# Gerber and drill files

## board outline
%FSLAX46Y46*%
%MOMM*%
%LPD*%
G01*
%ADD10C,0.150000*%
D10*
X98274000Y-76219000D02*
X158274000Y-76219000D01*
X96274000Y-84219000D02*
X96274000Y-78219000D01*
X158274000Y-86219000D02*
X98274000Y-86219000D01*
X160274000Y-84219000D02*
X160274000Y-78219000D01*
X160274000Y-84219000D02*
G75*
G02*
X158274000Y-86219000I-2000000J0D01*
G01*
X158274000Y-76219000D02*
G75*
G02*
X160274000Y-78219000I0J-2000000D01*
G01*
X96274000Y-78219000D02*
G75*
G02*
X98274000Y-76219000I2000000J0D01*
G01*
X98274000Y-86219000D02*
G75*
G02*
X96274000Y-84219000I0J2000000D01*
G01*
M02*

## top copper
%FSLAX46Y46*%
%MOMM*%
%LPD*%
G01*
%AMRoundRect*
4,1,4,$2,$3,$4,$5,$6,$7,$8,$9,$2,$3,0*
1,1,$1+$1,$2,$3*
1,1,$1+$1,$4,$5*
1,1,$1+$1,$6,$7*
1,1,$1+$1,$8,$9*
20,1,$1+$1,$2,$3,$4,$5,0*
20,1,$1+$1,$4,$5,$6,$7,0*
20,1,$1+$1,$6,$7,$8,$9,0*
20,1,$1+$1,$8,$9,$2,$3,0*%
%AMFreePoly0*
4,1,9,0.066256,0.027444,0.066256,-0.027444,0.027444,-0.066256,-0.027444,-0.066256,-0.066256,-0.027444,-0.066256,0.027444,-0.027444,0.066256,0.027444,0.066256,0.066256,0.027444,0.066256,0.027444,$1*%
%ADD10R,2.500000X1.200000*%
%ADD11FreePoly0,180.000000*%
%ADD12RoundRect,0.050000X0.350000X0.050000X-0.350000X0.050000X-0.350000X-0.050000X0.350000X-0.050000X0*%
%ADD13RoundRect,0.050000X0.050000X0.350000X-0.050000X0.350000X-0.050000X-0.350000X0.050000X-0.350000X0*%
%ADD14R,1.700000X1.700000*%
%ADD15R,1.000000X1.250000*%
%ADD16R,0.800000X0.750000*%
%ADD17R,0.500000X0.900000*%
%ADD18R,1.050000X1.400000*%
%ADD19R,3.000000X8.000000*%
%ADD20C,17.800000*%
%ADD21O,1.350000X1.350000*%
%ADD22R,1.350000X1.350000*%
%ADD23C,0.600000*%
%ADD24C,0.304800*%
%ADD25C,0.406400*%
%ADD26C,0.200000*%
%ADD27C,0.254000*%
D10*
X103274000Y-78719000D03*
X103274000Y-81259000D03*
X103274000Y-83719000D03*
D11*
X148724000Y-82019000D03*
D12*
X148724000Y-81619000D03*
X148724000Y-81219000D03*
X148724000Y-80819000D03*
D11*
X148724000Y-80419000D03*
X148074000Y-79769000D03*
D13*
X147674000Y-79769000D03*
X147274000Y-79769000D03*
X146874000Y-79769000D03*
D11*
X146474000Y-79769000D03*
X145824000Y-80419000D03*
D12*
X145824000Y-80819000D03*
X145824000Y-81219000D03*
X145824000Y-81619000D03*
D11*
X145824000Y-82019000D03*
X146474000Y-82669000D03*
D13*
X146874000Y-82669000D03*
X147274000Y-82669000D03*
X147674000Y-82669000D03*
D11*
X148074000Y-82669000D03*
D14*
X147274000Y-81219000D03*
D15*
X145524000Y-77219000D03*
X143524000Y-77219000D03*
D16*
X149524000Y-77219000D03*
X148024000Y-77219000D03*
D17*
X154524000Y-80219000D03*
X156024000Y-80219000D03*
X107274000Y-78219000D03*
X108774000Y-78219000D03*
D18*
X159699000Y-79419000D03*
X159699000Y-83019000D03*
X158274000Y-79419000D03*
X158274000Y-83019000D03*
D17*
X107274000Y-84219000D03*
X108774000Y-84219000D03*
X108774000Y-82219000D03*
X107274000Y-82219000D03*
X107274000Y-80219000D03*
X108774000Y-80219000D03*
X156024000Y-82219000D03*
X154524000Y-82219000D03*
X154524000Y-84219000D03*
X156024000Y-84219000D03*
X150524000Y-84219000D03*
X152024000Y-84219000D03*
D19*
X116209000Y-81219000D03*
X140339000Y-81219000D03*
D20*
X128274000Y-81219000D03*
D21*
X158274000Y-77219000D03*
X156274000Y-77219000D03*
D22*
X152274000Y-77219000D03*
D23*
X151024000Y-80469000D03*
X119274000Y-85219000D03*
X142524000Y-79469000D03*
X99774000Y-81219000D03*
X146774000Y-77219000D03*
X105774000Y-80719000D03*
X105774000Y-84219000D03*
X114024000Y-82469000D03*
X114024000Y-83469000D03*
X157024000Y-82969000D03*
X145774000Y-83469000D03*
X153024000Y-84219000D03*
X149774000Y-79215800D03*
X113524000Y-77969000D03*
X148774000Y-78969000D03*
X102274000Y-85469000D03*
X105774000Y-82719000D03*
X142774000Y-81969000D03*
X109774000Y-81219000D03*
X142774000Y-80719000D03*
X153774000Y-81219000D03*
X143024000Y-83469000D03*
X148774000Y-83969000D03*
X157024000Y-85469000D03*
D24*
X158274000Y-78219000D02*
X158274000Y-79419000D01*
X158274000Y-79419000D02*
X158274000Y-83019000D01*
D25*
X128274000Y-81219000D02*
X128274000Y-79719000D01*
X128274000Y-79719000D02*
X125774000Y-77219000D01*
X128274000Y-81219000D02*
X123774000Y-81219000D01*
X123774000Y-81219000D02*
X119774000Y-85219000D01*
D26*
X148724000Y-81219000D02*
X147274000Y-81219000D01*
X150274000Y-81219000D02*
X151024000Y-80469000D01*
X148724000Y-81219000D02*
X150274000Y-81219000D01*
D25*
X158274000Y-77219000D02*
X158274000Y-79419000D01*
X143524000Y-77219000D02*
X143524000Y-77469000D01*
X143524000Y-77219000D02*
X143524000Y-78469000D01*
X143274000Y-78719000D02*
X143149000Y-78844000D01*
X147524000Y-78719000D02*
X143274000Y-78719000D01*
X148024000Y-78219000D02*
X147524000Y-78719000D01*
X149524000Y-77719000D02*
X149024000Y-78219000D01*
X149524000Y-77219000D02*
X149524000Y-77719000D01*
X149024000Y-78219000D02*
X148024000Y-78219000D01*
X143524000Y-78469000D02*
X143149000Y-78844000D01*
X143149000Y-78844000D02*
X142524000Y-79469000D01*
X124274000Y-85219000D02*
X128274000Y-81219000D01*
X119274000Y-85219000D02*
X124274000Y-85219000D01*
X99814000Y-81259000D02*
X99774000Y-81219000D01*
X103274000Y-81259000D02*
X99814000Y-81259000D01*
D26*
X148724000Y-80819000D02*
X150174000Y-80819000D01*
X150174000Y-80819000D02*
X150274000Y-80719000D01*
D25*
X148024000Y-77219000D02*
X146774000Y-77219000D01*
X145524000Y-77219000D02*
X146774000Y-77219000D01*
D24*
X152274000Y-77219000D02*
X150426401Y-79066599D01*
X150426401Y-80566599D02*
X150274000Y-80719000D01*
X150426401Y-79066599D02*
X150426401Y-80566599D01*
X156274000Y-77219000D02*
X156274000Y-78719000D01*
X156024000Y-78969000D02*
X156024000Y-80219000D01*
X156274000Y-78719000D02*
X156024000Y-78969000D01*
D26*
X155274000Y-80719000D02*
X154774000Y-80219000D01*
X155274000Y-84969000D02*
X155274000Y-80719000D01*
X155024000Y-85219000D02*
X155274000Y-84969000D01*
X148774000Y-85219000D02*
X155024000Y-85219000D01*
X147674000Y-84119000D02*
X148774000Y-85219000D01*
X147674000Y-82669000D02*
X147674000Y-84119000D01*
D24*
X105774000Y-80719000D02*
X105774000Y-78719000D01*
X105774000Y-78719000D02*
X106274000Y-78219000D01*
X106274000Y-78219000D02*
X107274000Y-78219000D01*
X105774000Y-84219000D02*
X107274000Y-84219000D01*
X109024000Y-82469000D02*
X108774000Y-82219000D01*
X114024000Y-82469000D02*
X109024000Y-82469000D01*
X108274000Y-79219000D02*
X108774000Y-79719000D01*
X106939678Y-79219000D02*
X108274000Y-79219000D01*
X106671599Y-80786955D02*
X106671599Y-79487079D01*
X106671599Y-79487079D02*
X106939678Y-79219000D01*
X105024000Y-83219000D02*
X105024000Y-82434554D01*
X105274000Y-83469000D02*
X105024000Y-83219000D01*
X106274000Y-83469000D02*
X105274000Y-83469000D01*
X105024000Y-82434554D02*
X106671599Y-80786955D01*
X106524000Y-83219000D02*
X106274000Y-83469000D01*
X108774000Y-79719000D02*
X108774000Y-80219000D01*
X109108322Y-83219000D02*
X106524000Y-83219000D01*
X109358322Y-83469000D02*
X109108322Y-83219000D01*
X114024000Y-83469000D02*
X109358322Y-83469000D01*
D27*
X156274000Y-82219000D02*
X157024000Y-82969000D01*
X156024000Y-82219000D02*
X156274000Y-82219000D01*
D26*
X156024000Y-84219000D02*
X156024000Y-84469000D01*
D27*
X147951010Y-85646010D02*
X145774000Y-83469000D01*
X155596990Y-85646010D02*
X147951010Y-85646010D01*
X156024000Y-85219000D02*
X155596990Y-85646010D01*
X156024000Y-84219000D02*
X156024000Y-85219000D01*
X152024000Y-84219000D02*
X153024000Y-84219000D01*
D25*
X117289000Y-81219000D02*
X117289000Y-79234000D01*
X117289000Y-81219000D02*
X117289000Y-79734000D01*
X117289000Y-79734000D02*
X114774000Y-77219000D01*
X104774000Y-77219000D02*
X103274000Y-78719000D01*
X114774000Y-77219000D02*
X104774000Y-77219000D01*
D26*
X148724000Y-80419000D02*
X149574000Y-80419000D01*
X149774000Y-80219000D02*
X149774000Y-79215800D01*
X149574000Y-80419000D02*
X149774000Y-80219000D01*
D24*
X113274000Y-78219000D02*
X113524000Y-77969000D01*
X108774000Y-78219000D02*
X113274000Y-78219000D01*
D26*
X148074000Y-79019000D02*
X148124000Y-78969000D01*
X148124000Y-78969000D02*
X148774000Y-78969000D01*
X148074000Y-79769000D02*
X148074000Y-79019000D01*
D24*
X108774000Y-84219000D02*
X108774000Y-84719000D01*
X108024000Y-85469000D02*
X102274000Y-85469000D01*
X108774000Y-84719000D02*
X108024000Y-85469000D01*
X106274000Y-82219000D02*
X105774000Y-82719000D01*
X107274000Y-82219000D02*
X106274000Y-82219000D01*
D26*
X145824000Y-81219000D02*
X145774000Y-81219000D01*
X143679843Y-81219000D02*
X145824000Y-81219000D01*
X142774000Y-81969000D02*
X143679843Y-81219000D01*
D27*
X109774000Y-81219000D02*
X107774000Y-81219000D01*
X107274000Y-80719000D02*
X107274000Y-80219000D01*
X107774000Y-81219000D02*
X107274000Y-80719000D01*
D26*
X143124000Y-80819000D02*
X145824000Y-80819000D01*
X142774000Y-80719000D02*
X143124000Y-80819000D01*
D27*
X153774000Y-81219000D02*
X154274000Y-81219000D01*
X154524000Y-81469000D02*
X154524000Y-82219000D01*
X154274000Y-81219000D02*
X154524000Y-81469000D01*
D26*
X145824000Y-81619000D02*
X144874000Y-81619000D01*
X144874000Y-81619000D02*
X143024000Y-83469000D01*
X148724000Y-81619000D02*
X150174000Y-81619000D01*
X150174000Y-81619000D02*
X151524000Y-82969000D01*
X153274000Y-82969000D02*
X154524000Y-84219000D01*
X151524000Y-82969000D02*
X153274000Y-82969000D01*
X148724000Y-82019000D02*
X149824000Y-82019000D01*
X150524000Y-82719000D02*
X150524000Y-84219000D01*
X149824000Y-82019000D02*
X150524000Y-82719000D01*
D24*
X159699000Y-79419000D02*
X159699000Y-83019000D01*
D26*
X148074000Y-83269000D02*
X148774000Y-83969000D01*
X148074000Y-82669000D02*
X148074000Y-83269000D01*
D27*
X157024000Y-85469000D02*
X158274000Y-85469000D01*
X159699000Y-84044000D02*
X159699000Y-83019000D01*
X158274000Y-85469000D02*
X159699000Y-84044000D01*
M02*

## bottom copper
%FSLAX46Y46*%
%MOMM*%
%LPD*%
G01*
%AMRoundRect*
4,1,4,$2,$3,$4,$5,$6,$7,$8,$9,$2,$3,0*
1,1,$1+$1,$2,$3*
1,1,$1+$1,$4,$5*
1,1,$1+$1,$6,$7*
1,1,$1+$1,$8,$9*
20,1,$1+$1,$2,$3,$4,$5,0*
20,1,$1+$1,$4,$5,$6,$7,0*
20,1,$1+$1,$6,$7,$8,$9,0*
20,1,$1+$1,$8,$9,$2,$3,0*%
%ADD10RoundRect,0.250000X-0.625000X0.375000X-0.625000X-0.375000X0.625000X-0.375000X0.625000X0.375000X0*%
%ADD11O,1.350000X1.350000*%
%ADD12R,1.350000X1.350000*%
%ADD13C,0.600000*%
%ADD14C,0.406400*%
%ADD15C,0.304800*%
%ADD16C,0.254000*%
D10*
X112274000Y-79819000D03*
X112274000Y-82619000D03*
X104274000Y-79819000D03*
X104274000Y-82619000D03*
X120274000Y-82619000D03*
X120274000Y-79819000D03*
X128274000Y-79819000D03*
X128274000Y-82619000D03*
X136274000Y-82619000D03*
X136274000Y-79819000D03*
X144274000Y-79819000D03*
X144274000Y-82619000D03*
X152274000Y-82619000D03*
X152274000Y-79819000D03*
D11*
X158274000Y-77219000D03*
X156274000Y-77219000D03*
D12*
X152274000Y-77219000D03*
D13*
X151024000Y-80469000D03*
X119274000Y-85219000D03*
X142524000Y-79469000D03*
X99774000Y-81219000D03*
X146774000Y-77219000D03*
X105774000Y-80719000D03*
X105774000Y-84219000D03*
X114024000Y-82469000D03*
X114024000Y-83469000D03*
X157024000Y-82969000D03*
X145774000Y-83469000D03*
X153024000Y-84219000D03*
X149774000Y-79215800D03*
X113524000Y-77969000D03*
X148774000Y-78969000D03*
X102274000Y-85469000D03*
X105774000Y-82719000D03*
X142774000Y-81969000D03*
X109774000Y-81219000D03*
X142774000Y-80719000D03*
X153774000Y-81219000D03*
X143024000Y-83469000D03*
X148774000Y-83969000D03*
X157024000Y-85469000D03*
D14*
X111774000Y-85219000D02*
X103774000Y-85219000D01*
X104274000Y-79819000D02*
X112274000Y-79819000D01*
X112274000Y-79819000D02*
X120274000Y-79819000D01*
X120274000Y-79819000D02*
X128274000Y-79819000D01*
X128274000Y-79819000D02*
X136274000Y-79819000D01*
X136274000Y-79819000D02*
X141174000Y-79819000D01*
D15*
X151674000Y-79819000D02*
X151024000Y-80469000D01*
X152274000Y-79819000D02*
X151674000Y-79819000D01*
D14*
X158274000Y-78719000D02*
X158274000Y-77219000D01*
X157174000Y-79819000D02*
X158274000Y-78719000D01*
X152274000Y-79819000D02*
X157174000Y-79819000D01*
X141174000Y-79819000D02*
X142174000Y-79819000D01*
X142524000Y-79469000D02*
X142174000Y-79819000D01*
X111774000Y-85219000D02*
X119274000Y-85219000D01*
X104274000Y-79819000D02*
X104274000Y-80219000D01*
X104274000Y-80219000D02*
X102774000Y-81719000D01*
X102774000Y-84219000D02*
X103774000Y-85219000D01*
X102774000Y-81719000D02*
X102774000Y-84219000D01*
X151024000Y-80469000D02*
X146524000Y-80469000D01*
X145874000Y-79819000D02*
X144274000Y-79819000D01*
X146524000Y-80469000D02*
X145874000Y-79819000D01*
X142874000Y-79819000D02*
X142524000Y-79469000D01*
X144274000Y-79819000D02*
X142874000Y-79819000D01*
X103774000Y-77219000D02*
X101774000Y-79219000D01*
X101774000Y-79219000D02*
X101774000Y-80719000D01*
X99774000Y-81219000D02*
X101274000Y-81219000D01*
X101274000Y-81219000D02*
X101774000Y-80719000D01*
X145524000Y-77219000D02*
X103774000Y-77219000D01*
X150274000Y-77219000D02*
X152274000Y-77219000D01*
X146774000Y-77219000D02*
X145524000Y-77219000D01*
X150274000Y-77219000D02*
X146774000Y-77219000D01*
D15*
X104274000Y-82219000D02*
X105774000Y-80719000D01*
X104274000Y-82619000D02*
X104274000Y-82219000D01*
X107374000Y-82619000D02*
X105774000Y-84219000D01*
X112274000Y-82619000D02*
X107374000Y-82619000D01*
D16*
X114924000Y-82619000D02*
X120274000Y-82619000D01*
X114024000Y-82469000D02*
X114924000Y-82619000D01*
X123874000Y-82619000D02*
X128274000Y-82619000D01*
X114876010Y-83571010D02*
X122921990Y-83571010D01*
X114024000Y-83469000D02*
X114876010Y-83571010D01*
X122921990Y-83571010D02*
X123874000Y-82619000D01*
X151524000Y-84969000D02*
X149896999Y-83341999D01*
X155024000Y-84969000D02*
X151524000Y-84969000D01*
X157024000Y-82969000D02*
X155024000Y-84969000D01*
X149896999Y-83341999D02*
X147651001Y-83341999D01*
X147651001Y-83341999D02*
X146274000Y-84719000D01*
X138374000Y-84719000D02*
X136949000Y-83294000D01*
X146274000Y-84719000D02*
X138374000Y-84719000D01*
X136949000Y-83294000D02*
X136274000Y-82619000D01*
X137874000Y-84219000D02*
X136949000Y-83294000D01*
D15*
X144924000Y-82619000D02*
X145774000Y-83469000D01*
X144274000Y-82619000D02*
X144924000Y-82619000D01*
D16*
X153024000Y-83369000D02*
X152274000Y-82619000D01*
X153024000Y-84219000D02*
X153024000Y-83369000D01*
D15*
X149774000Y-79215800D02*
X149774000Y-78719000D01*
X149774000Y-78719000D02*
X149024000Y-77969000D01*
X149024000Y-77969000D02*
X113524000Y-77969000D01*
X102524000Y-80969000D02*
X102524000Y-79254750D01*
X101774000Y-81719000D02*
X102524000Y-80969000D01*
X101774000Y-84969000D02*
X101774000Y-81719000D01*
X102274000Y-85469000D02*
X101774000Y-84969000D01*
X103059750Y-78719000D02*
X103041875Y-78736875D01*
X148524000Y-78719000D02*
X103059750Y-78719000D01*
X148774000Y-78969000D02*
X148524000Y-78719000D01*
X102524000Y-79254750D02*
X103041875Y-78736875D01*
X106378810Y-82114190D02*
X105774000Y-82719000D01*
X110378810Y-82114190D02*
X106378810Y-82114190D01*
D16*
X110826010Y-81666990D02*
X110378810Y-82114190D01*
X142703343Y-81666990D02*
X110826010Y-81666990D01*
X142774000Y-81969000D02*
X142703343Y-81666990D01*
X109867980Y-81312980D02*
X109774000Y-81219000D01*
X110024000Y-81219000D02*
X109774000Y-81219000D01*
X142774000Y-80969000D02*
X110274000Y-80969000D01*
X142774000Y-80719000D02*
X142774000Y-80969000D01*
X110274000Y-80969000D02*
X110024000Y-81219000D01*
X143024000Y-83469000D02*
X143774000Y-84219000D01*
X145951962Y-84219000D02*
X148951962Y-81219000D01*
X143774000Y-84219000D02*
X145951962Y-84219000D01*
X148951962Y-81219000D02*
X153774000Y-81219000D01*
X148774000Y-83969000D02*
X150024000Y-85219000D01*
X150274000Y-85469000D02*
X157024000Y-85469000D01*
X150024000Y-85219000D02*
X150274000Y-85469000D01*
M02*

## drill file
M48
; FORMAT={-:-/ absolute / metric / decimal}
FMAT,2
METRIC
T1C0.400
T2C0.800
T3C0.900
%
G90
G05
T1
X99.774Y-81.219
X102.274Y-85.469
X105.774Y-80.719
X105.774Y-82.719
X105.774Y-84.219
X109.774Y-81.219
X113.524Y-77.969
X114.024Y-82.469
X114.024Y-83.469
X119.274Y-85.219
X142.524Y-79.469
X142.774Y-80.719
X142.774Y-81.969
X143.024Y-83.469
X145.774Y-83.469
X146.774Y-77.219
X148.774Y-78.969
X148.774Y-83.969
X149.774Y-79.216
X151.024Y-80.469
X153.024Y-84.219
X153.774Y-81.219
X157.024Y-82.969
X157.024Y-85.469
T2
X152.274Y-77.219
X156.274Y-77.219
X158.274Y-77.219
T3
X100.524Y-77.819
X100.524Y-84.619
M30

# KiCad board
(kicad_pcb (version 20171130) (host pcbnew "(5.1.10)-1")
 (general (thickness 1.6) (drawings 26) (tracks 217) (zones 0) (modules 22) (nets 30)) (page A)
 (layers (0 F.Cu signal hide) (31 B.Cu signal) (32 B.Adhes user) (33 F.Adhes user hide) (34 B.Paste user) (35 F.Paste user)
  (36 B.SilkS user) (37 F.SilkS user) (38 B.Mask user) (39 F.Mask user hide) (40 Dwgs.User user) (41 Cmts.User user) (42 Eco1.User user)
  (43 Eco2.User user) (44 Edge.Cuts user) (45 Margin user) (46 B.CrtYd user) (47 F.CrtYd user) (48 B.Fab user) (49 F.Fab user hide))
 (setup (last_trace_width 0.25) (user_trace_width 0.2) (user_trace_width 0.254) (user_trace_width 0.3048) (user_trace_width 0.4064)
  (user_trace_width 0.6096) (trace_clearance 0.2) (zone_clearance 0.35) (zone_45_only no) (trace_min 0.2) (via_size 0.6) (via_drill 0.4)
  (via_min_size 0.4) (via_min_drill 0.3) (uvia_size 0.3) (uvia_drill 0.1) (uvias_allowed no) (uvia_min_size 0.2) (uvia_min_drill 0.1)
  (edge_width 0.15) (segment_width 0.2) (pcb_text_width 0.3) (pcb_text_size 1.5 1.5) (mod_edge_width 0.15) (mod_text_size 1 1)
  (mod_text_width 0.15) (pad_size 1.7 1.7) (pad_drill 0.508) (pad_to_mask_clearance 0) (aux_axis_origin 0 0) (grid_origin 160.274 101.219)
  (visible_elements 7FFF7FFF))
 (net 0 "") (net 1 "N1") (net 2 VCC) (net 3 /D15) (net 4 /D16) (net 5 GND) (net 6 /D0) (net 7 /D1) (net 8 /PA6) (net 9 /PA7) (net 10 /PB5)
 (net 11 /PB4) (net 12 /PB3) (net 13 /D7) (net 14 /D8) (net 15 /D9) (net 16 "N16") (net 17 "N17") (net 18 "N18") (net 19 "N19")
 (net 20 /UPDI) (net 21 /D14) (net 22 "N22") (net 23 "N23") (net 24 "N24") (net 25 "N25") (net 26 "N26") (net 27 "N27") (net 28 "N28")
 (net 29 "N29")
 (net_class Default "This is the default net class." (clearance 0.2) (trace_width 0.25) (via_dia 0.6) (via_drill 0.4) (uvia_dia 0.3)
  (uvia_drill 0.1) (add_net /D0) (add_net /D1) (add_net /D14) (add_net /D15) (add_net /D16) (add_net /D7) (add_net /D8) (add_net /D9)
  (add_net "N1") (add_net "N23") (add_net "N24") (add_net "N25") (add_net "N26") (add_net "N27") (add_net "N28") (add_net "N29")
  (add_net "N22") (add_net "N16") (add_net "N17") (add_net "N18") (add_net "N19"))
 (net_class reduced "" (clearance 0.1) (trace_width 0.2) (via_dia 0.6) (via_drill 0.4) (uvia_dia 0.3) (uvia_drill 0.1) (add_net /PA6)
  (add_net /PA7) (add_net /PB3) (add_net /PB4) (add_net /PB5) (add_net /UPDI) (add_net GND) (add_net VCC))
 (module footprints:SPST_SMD (layer F.Cu) (at 103.274 81.219 270)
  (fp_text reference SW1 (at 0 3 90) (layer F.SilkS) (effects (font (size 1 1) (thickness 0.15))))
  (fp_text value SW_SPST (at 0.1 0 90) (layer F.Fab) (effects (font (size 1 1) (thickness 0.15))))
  (pad "" np_thru_hole circle (at 3.4 2.75 270) (size 0.9 0.9) (drill 0.9) (layers *.Cu *.Mask))
  (pad 1 smd rect (at -2.5 0 270) (size 1.2 2.5) (layers F.Cu F.Paste F.Mask) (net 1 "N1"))
  (pad 2 smd rect (at 0.04 0 270) (size 1.2 2.5) (layers F.Cu F.Paste F.Mask) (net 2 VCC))
  (pad 3 smd rect (at 2.5 0 270) (size 1.2 2.5) (layers F.Cu F.Paste F.Mask))
  (pad "" np_thru_hole circle (at -3.4 2.75 270) (size 0.9 0.9) (drill 0.9) (layers *.Cu *.Mask)))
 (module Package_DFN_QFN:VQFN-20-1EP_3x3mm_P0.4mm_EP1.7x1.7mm (layer F.Cu) (at 147.274 81.219 180)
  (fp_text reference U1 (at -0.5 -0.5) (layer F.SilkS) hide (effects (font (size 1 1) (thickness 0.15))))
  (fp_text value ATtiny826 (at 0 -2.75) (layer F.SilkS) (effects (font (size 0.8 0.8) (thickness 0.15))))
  (pad 1 smd custom (at -1.45 -0.8 180) (size 0.143431 0.143431) (layers F.Cu F.Paste F.Mask) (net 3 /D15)
   (options (clearance outline) (anchor circle)) (primitives))
  (pad 2 smd roundrect (at -1.45 -0.4 180) (size 0.8 0.2) (layers F.Cu F.Paste F.Mask) (roundrect_rratio 0.25) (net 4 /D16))
  (pad 3 smd roundrect (at -1.45 0 180) (size 0.8 0.2) (layers F.Cu F.Paste F.Mask) (roundrect_rratio 0.25) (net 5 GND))
  (pad 4 smd roundrect (at -1.45 0.4 180) (size 0.8 0.2) (layers F.Cu F.Paste F.Mask) (roundrect_rratio 0.25) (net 2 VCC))
  (pad 5 smd custom (at -1.45 0.8 180) (size 0.143431 0.143431) (layers F.Cu F.Paste F.Mask) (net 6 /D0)
   (options (clearance outline) (anchor circle)) (primitives))
  (pad 6 smd custom (at -0.8 1.45 180) (size 0.143431 0.143431) (layers F.Cu F.Paste F.Mask) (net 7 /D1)
   (options (clearance outline) (anchor circle)) (primitives))
  (pad 7 smd roundrect (at -0.4 1.45 180) (size 0.2 0.8) (layers F.Cu F.Paste F.Mask) (roundrect_rratio 0.25) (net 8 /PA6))
  (pad 8 smd roundrect (at 0 1.45 180) (size 0.2 0.8) (layers F.Cu F.Paste F.Mask) (roundrect_rratio 0.25) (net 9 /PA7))
  (pad 9 smd roundrect (at 0.4 1.45 180) (size 0.2 0.8) (layers F.Cu F.Paste F.Mask) (roundrect_rratio 0.25) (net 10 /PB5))
  (pad 10 smd custom (at 0.8 1.45 180) (size 0.143431 0.143431) (layers F.Cu F.Paste F.Mask) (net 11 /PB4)
   (options (clearance outline) (anchor circle)) (primitives))
  (pad 11 smd custom (at 1.45 0.8 180) (size 0.143431 0.143431) (layers F.Cu F.Paste F.Mask) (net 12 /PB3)
   (options (clearance outline) (anchor circle)) (primitives))
  (pad 12 smd roundrect (at 1.45 0.4 180) (size 0.8 0.2) (layers F.Cu F.Paste F.Mask) (roundrect_rratio 0.25) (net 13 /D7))
  (pad 13 smd roundrect (at 1.45 0 180) (size 0.8 0.2) (layers F.Cu F.Paste F.Mask) (roundrect_rratio 0.25) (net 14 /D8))
  (pad 14 smd roundrect (at 1.45 -0.4 180) (size 0.8 0.2) (layers F.Cu F.Paste F.Mask) (roundrect_rratio 0.25) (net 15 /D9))
  (pad 15 smd custom (at 1.45 -0.8 180) (size 0.143431 0.143431) (layers F.Cu F.Paste F.Mask) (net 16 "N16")
   (options (clearance outline) (anchor circle)) (primitives))
  (pad 16 smd custom (at 0.8 -1.45 180) (size 0.143431 0.143431) (layers F.Cu F.Paste F.Mask) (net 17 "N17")
   (options (clearance outline) (anchor circle)) (primitives))
  (pad 17 smd roundrect (at 0.4 -1.45 180) (size 0.2 0.8) (layers F.Cu F.Paste F.Mask) (roundrect_rratio 0.25) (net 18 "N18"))
  (pad 18 smd roundrect (at 0 -1.45 180) (size 0.2 0.8) (layers F.Cu F.Paste F.Mask) (roundrect_rratio 0.25) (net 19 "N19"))
  (pad 19 smd roundrect (at -0.4 -1.45 180) (size 0.2 0.8) (layers F.Cu F.Paste F.Mask) (roundrect_rratio 0.25) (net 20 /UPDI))
  (pad 20 smd custom (at -0.8 -1.45 180) (size 0.143431 0.143431) (layers F.Cu F.Paste F.Mask) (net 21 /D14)
   (options (clearance outline) (anchor circle)) (primitives))
  (pad 21 smd rect (at 0 0 180) (size 1.7 1.7) (layers F.Cu F.Mask) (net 5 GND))
  (pad "" smd roundrect (at -0.425 -0.425 180) (size 0.69 0.69) (layers F.Paste) (roundrect_rratio 0.25))
  (pad "" smd roundrect (at -0.425 0.425 180) (size 0.69 0.69) (layers F.Paste) (roundrect_rratio 0.25))
  (pad "" smd roundrect (at 0.425 -0.425 180) (size 0.69 0.69) (layers F.Paste) (roundrect_rratio 0.25))
  (pad "" smd roundrect (at 0.425 0.425 180) (size 0.69 0.69) (layers F.Paste) (roundrect_rratio 0.25)))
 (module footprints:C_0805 (layer F.Cu) (at 144.524 77.219 180)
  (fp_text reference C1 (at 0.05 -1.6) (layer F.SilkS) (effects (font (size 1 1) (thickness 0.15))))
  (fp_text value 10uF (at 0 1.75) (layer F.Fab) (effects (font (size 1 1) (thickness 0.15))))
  (pad 1 smd rect (at -1 0 180) (size 1 1.25) (layers F.Cu F.Paste F.Mask) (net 2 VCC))
  (pad 2 smd rect (at 1 0 180) (size 1 1.25) (layers F.Cu F.Paste F.Mask) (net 5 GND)))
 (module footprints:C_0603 (layer F.Cu) (at 148.774 77.219)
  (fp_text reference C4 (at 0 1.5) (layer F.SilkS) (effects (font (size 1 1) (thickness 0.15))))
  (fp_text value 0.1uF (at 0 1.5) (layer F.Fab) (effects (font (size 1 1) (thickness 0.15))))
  (pad 2 smd rect (at 0.75 0) (size 0.8 0.75) (layers F.Cu F.Paste F.Mask) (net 5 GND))
  (pad 1 smd rect (at -0.75 0) (size 0.8 0.75) (layers F.Cu F.Paste F.Mask) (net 2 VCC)))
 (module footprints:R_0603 (layer F.Cu) (at 155.274 80.219)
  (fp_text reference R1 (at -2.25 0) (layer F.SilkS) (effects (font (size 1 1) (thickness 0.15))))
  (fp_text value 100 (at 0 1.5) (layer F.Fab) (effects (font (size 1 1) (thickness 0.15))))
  (pad 1 smd rect (at -0.75 0) (size 0.5 0.9) (layers F.Cu F.Paste F.Mask) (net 20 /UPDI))
  (pad 2 smd rect (at 0.75 0) (size 0.5 0.9) (layers F.Cu F.Paste F.Mask) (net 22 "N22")))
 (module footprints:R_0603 (layer F.Cu) (at 108.024 78.219 180)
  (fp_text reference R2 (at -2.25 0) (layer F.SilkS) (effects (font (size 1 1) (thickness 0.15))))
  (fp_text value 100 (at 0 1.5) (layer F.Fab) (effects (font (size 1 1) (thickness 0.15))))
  (pad 2 smd rect (at 0.75 0 180) (size 0.5 0.9) (layers F.Cu F.Paste F.Mask) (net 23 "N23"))
  (pad 1 smd rect (at -0.75 0 180) (size 0.5 0.9) (layers F.Cu F.Paste F.Mask) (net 6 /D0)))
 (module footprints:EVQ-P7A (layer F.Cu) (at 158.974 81.219 90)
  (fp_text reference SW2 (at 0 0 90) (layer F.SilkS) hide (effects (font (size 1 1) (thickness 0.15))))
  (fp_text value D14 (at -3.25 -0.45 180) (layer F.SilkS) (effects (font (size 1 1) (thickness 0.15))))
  (pad 2 smd rect (at 1.8 0.725 90) (size 1.4 1.05) (layers F.Cu F.Paste F.Mask) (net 21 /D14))
  (pad 2 smd rect (at -1.8 0.725 90) (size 1.4 1.05) (layers F.Cu F.Paste F.Mask) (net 21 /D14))
  (pad 1 smd rect (at 1.8 -0.7 90) (size 1.4 1.05) (layers F.Cu F.Paste F.Mask) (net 5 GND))
  (pad 1 smd rect (at -1.8 -0.7 90) (size 1.4 1.05) (layers F.Cu F.Paste F.Mask) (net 5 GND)))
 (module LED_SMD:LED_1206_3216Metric (layer B.Cu) (at 112.274 81.219 270)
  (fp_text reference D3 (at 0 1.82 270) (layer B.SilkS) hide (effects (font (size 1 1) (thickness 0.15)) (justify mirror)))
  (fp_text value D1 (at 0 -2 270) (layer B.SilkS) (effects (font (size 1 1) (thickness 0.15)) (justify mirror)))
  (pad 1 smd roundrect (at -1.4 0 270) (size 1.25 1.75) (layers B.Cu B.Paste B.Mask) (roundrect_rratio 0.2) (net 5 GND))
  (pad 2 smd roundrect (at 1.4 0 270) (size 1.25 1.75) (layers B.Cu B.Paste B.Mask) (roundrect_rratio 0.2) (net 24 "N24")))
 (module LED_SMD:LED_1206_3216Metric (layer B.Cu) (at 104.274 81.219 270)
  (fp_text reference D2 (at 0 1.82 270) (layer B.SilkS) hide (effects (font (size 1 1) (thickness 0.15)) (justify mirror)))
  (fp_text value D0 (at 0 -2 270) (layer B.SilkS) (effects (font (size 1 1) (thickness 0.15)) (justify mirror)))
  (pad 1 smd roundrect (at -1.4 0 270) (size 1.25 1.75) (layers B.Cu B.Paste B.Mask) (roundrect_rratio 0.2) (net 5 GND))
  (pad 2 smd roundrect (at 1.4 0 270) (size 1.25 1.75) (layers B.Cu B.Paste B.Mask) (roundrect_rratio 0.2) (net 23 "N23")))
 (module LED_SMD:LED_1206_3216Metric (layer B.Cu) (at 120.274 81.219 270)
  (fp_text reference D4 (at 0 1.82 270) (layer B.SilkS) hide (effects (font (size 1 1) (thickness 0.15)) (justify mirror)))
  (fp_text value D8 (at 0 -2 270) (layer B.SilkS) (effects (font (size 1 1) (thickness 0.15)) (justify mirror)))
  (pad 2 smd roundrect (at 1.4 0 270) (size 1.25 1.75) (layers B.Cu B.Paste B.Mask) (roundrect_rratio 0.2) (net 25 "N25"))
  (pad 1 smd roundrect (at -1.4 0 270) (size 1.25 1.75) (layers B.Cu B.Paste B.Mask) (roundrect_rratio 0.2) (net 5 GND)))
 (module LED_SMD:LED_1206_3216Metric (layer B.Cu) (at 128.274 81.219 270)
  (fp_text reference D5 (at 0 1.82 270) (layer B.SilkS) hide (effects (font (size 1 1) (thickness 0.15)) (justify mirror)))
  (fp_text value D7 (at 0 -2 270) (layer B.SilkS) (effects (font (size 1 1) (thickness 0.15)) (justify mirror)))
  (pad 1 smd roundrect (at -1.4 0 270) (size 1.25 1.75) (layers B.Cu B.Paste B.Mask) (roundrect_rratio 0.2) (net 5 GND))
  (pad 2 smd roundrect (at 1.4 0 270) (size 1.25 1.75) (layers B.Cu B.Paste B.Mask) (roundrect_rratio 0.2) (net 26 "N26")))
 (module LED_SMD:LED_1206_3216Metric (layer B.Cu) (at 136.274 81.219 270)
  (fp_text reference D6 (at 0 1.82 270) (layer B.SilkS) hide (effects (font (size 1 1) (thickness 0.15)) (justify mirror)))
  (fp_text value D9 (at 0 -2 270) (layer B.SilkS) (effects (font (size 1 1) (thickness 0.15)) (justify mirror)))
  (pad 2 smd roundrect (at 1.4 0 270) (size 1.25 1.75) (layers B.Cu B.Paste B.Mask) (roundrect_rratio 0.2) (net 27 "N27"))
  (pad 1 smd roundrect (at -1.4 0 270) (size 1.25 1.75) (layers B.Cu B.Paste B.Mask) (roundrect_rratio 0.2) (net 5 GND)))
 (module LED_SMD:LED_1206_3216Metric (layer B.Cu) (at 144.274 81.219 270)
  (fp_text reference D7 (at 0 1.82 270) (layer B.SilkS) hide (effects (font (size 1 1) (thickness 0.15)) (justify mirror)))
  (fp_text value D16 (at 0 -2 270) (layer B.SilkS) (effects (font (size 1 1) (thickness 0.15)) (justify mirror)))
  (pad 1 smd roundrect (at -1.4 0 270) (size 1.25 1.75) (layers B.Cu B.Paste B.Mask) (roundrect_rratio 0.2) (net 5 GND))
  (pad 2 smd roundrect (at 1.4 0 270) (size 1.25 1.75) (layers B.Cu B.Paste B.Mask) (roundrect_rratio 0.2) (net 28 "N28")))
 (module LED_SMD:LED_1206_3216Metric (layer B.Cu) (at 152.274 81.219 270)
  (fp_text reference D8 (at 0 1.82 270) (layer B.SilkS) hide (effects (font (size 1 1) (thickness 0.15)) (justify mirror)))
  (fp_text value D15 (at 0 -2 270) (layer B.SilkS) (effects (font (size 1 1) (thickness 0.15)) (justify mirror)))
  (pad 2 smd roundrect (at 1.4 0 270) (size 1.25 1.75) (layers B.Cu B.Paste B.Mask) (roundrect_rratio 0.2) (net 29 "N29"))
  (pad 1 smd roundrect (at -1.4 0 270) (size 1.25 1.75) (layers B.Cu B.Paste B.Mask) (roundrect_rratio 0.2) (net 5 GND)))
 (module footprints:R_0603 (layer F.Cu) (at 108.024 84.219 180)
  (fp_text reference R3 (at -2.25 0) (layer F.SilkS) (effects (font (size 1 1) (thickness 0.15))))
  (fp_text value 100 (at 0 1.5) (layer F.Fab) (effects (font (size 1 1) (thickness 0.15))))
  (pad 2 smd rect (at 0.75 0 180) (size 0.5 0.9) (layers F.Cu F.Paste F.Mask) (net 24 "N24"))
  (pad 1 smd rect (at -0.75 0 180) (size 0.5 0.9) (layers F.Cu F.Paste F.Mask) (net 7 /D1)))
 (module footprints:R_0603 (layer F.Cu) (at 108.024 82.219)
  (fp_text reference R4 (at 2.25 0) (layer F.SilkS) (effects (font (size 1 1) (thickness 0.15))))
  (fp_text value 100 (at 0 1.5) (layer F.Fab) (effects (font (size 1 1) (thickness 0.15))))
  (pad 2 smd rect (at 0.75 0) (size 0.5 0.9) (layers F.Cu F.Paste F.Mask) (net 25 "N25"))
  (pad 1 smd rect (at -0.75 0) (size 0.5 0.9) (layers F.Cu F.Paste F.Mask) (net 14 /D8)))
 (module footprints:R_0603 (layer F.Cu) (at 108.024 80.219)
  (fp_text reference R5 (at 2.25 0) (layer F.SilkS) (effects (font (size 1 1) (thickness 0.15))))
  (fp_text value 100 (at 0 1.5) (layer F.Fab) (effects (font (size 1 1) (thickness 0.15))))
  (pad 1 smd rect (at -0.75 0) (size 0.5 0.9) (layers F.Cu F.Paste F.Mask) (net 13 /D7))
  (pad 2 smd rect (at 0.75 0) (size 0.5 0.9) (layers F.Cu F.Paste F.Mask) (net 26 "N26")))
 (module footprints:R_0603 (layer F.Cu) (at 155.274 82.219)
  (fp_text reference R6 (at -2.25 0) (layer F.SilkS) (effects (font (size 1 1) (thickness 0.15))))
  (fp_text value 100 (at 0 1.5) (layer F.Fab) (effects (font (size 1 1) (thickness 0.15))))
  (pad 2 smd rect (at 0.75 0) (size 0.5 0.9) (layers F.Cu F.Paste F.Mask) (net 27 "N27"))
  (pad 1 smd rect (at -0.75 0) (size 0.5 0.9) (layers F.Cu F.Paste F.Mask) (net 15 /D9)))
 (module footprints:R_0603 (layer F.Cu) (at 155.274 84.219)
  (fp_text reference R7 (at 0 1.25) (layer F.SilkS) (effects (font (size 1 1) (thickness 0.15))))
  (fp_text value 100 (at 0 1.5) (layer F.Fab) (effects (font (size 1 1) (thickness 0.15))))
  (pad 1 smd rect (at -0.75 0) (size 0.5 0.9) (layers F.Cu F.Paste F.Mask) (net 4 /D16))
  (pad 2 smd rect (at 0.75 0) (size 0.5 0.9) (layers F.Cu F.Paste F.Mask) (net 28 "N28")))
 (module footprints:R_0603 (layer F.Cu) (at 151.274 84.219)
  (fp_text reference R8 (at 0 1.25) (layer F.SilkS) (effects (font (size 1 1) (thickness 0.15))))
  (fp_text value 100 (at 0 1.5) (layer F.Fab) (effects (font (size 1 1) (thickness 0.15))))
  (pad 1 smd rect (at -0.75 0) (size 0.5 0.9) (layers F.Cu F.Paste F.Mask) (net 3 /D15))
  (pad 2 smd rect (at 0.75 0) (size 0.5 0.9) (layers F.Cu F.Paste F.Mask) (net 29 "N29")))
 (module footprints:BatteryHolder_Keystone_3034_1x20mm (layer F.Cu) (at 128.274 81.219)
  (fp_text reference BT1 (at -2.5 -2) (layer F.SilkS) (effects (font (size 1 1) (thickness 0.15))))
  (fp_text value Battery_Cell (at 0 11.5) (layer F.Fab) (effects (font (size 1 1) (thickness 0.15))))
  (pad 1 smd rect (at -12.065 0) (size 3 8) (layers F.Cu F.Paste F.Mask) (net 1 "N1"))
  (pad 1 smd rect (at 12.065 0) (size 3 8) (layers F.Cu F.Paste F.Mask) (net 1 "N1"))
  (pad 2 smd circle (at 0 0) (size 17.8 17.8) (layers F.Cu F.Mask) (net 5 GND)))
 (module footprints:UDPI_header (layer F.Cu) (at 152.274 77.219 90)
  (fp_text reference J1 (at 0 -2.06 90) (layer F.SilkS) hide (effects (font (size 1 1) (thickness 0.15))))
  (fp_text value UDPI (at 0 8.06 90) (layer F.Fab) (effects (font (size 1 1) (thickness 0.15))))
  (pad 4 thru_hole oval (at 0 6 90) (size 1.35 1.35) (drill 0.8) (layers *.Cu *.Mask) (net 5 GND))
  (pad 3 thru_hole oval (at 0 4 90) (size 1.35 1.35) (drill 0.8) (layers *.Cu *.Mask) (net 22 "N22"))
  (pad 1 thru_hole rect (at 0 0 90) (size 1.35 1.35) (drill 0.8) (layers *.Cu *.Mask) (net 2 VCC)))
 (gr_line (start 98.274 76.219) (end 158.274 76.219) (layer Edge.Cuts) (width 0.15))
 (gr_line (start 96.274 84.219) (end 96.274 78.219) (layer Edge.Cuts) (width 0.15))
 (gr_line (start 158.274 86.219) (end 98.274 86.219) (layer Edge.Cuts) (width 0.15))
 (gr_line (start 160.274 84.219) (end 160.274 78.219) (layer Edge.Cuts) (width 0.15))
 (gr_arc (start 158.274 84.219) (end 158.274 86.219) (angle -90) (layer Edge.Cuts) (width 0.15))
 (gr_arc (start 158.274 78.219) (end 160.274 78.219) (angle -90) (layer Edge.Cuts) (width 0.15))
 (gr_arc (start 98.274 78.219) (end 98.274 76.219) (angle -90) (layer Edge.Cuts) (width 0.15))
 (gr_arc (start 98.274 84.219) (end 96.274 84.219) (angle -90) (layer Edge.Cuts) (width 0.15))
 (segment (start 158.274 78.219) (end 158.274 79.419) (width 0.3048) (layer F.Cu) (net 5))
 (segment (start 158.274 79.419) (end 158.274 83.019) (width 0.3048) (layer F.Cu) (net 5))
 (segment (start 128.274 81.219) (end 128.274 79.719) (width 0.4064) (layer F.Cu) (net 5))
 (segment (start 128.274 79.719) (end 125.774 77.219) (width 0.4064) (layer F.Cu) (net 5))
 (segment (start 128.274 81.219) (end 123.774 81.219) (width 0.4064) (layer F.Cu) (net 5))
 (segment (start 123.774 81.219) (end 119.774 85.219) (width 0.4064) (layer F.Cu) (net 5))
 (segment (start 111.774 85.219) (end 103.774 85.219) (width 0.4064) (layer B.Cu) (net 5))
 (segment (start 104.274 79.819) (end 112.274 79.819) (width 0.4064) (layer B.Cu) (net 5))
 (segment (start 112.274 79.819) (end 120.274 79.819) (width 0.4064) (layer B.Cu) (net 5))
 (segment (start 120.274 79.819) (end 128.274 79.819) (width 0.4064) (layer B.Cu) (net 5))
 (segment (start 128.274 79.819) (end 136.274 79.819) (width 0.4064) (layer B.Cu) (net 5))
 (segment (start 136.274 79.819) (end 141.174 79.819) (width 0.4064) (layer B.Cu) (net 5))
 (segment (start 148.724 81.219) (end 147.274 81.219) (width 0.2) (layer F.Cu) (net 5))
 (via (at 151.024 80.469) (size 0.6) (drill 0.4) (layers F.Cu B.Cu) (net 5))
 (segment (start 150.274 81.219) (end 151.024 80.469) (width 0.2) (layer F.Cu) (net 5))
 (segment (start 148.724 81.219) (end 150.274 81.219) (width 0.2) (layer F.Cu) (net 5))
 (segment (start 151.674 79.819) (end 151.024 80.469) (width 0.3048) (layer B.Cu) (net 5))
 (segment (start 152.274 79.819) (end 151.674 79.819) (width 0.3048) (layer B.Cu) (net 5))
 (segment (start 158.274 78.719) (end 158.274 77.219) (width 0.4064) (layer B.Cu) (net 5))
 (segment (start 157.174 79.819) (end 158.274 78.719) (width 0.4064) (layer B.Cu) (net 5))
 (segment (start 152.274 79.819) (end 157.174 79.819) (width 0.4064) (layer B.Cu) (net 5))
 (segment (start 158.274 77.219) (end 158.274 79.419) (width 0.4064) (layer F.Cu) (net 5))
 (segment (start 143.524 77.219) (end 143.524 77.469) (width 0.4064) (layer F.Cu) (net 5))
 (segment (start 143.524 77.219) (end 143.524 78.469) (width 0.4064) (layer F.Cu) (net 5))
 (segment (start 141.174 79.819) (end 142.174 79.819) (width 0.4064) (layer B.Cu) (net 5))
 (segment (start 143.274 78.719) (end 143.149 78.844) (width 0.4064) (layer F.Cu) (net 5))
 (segment (start 147.524 78.719) (end 143.274 78.719) (width 0.4064) (layer F.Cu) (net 5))
 (segment (start 148.024 78.219) (end 147.524 78.719) (width 0.4064) (layer F.Cu) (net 5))
 (segment (start 149.524 77.719) (end 149.024 78.219) (width 0.4064) (layer F.Cu) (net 5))
 (segment (start 149.524 77.219) (end 149.524 77.719) (width 0.4064) (layer F.Cu) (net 5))
 (segment (start 149.024 78.219) (end 148.024 78.219) (width 0.4064) (layer F.Cu) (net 5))
 (segment (start 143.524 78.469) (end 143.149 78.844) (width 0.4064) (layer F.Cu) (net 5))
 (segment (start 143.149 78.844) (end 142.524 79.469) (width 0.4064) (layer F.Cu) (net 5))
 (segment (start 142.524 79.469) (end 142.174 79.819) (width 0.4064) (layer B.Cu) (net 5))
 (via (at 119.274 85.219) (size 0.6) (drill 0.4) (layers F.Cu B.Cu) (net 5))
 (segment (start 111.774 85.219) (end 119.274 85.219) (width 0.4064) (layer B.Cu) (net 5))
 (segment (start 124.274 85.219) (end 128.274 81.219) (width 0.4064) (layer F.Cu) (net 5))
 (segment (start 119.274 85.219) (end 124.274 85.219) (width 0.4064) (layer F.Cu) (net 5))
 (segment (start 104.274 79.819) (end 104.274 80.219) (width 0.4064) (layer B.Cu) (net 5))
 (segment (start 104.274 80.219) (end 102.774 81.719) (width 0.4064) (layer B.Cu) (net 5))
 (segment (start 102.774 84.219) (end 103.774 85.219) (width 0.4064) (layer B.Cu) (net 5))
 (segment (start 102.774 81.719) (end 102.774 84.219) (width 0.4064) (layer B.Cu) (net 5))
 (via (at 142.524 79.469) (size 0.6) (drill 0.4) (layers F.Cu B.Cu) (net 5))
 (segment (start 151.024 80.469) (end 146.524 80.469) (width 0.4064) (layer B.Cu) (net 5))
 (segment (start 145.874 79.819) (end 144.274 79.819) (width 0.4064) (layer B.Cu) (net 5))
 (segment (start 146.524 80.469) (end 145.874 79.819) (width 0.4064) (layer B.Cu) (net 5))
 (segment (start 142.874 79.819) (end 142.524 79.469) (width 0.4064) (layer B.Cu) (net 5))
 (segment (start 144.274 79.819) (end 142.874 79.819) (width 0.4064) (layer B.Cu) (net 5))
 (segment (start 103.774 77.219) (end 101.774 79.219) (width 0.4064) (layer B.Cu) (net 2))
 (segment (start 101.774 79.219) (end 101.774 80.719) (width 0.4064) (layer B.Cu) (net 2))
 (via (at 99.774 81.219) (size 0.6) (drill 0.4) (layers F.Cu B.Cu) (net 2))
 (segment (start 99.814 81.259) (end 99.774 81.219) (width 0.4064) (layer F.Cu) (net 2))
 (segment (start 103.274 81.259) (end 99.814 81.259) (width 0.4064) (layer F.Cu) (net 2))
 (segment (start 99.774 81.219) (end 101.274 81.219) (width 0.4064) (layer B.Cu) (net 2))
 (segment (start 101.274 81.219) (end 101.774 80.719) (width 0.4064) (layer B.Cu) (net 2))
 (segment (start 148.724 80.819) (end 150.174 80.819) (width 0.2) (layer F.Cu) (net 2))
 (segment (start 150.174 80.819) (end 150.274 80.719) (width 0.2) (layer F.Cu) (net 2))
 (segment (start 145.524 77.219) (end 103.774 77.219) (width 0.4064) (layer B.Cu) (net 2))
 (segment (start 150.274 77.219) (end 152.274 77.219) (width 0.4064) (layer B.Cu) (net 2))
 (via (at 146.774 77.219) (size 0.6) (drill 0.4) (layers F.Cu B.Cu) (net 2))
 (segment (start 148.024 77.219) (end 146.774 77.219) (width 0.4064) (layer F.Cu) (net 2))
 (segment (start 146.774 77.219) (end 145.524 77.219) (width 0.4064) (layer B.Cu) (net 2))
 (segment (start 150.274 77.219) (end 146.774 77.219) (width 0.4064) (layer B.Cu) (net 2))
 (segment (start 145.524 77.219) (end 146.774 77.219) (width 0.4064) (layer F.Cu) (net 2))
 (segment (start 152.274 77.219) (end 150.426401 79.066599) (width 0.3048) (layer F.Cu) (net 2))
 (segment (start 150.426401 80.566599) (end 150.274 80.719) (width 0.3048) (layer F.Cu) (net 2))
 (segment (start 150.426401 79.066599) (end 150.426401 80.566599) (width 0.3048) (layer F.Cu) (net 2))
 (segment (start 156.274 77.219) (end 156.274 78.719) (width 0.3048) (layer F.Cu) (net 22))
 (segment (start 156.024 78.969) (end 156.024 80.219) (width 0.3048) (layer F.Cu) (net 22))
 (segment (start 156.274 78.719) (end 156.024 78.969) (width 0.3048) (layer F.Cu) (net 22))
 (segment (start 155.274 80.719) (end 154.774 80.219) (width 0.2) (layer F.Cu) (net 20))
 (segment (start 155.274 84.969) (end 155.274 80.719) (width 0.2) (layer F.Cu) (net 20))
 (segment (start 155.024 85.219) (end 155.274 84.969) (width 0.2) (layer F.Cu) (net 20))
 (segment (start 148.774 85.219) (end 155.024 85.219) (width 0.2) (layer F.Cu) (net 20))
 (segment (start 147.674 84.119) (end 148.774 85.219) (width 0.2) (layer F.Cu) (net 20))
 (segment (start 147.674 82.669) (end 147.674 84.119) (width 0.2) (layer F.Cu) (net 20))
 (via (at 105.774 80.719) (size 0.6) (drill 0.4) (layers F.Cu B.Cu) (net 23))
 (segment (start 104.274 82.219) (end 105.774 80.719) (width 0.3048) (layer B.Cu) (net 23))
 (segment (start 104.274 82.619) (end 104.274 82.219) (width 0.3048) (layer B.Cu) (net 23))
 (segment (start 105.774 80.719) (end 105.774 78.719) (width 0.3048) (layer F.Cu) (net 23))
 (segment (start 105.774 78.719) (end 106.274 78.219) (width 0.3048) (layer F.Cu) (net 23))
 (segment (start 106.274 78.219) (end 107.274 78.219) (width 0.3048) (layer F.Cu) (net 23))
 (via (at 105.774 84.219) (size 0.6) (drill 0.4) (layers F.Cu B.Cu) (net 24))
 (segment (start 107.374 82.619) (end 105.774 84.219) (width 0.3048) (layer B.Cu) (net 24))
 (segment (start 112.274 82.619) (end 107.374 82.619) (width 0.3048) (layer B.Cu) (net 24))
 (segment (start 105.774 84.219) (end 107.274 84.219) (width 0.3048) (layer F.Cu) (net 24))
 (segment (start 114.924 82.619) (end 120.274 82.619) (width 0.254) (layer B.Cu) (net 25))
 (segment (start 114.024 82.469) (end 114.924 82.619) (width 0.254) (layer B.Cu) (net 25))
 (via (at 114.024 82.469) (size 0.6) (drill 0.4) (layers F.Cu B.Cu) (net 25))
 (segment (start 109.024 82.469) (end 108.774 82.219) (width 0.3048) (layer F.Cu) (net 25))
 (segment (start 114.024 82.469) (end 109.024 82.469) (width 0.3048) (layer F.Cu) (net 25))
 (segment (start 123.874 82.619) (end 128.274 82.619) (width 0.254) (layer B.Cu) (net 26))
 (segment (start 114.87601 83.57101) (end 122.92199 83.57101) (width 0.254) (layer B.Cu) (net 26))
 (segment (start 114.024 83.469) (end 114.87601 83.57101) (width 0.254) (layer B.Cu) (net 26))
 (segment (start 122.92199 83.57101) (end 123.874 82.619) (width 0.254) (layer B.Cu) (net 26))
 (via (at 114.024 83.469) (size 0.6) (drill 0.4) (layers F.Cu B.Cu) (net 26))
 (segment (start 108.274 79.219) (end 108.774 79.719) (width 0.3048) (layer F.Cu) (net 26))
 (segment (start 106.939678 79.219) (end 108.274 79.219) (width 0.3048) (layer F.Cu) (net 26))
 (segment (start 106.671599 80.786955) (end 106.671599 79.487079) (width 0.3048) (layer F.Cu) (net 26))
 (segment (start 106.671599 79.487079) (end 106.939678 79.219) (width 0.3048) (layer F.Cu) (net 26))
 (segment (start 105.024 83.219) (end 105.024 82.434554) (width 0.3048) (layer F.Cu) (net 26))
 (segment (start 105.274 83.469) (end 105.024 83.219) (width 0.3048) (layer F.Cu) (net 26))
 (segment (start 106.274 83.469) (end 105.274 83.469) (width 0.3048) (layer F.Cu) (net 26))
 (segment (start 105.024 82.434554) (end 106.671599 80.786955) (width 0.3048) (layer F.Cu) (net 26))
 (segment (start 106.524 83.219) (end 106.274 83.469) (width 0.3048) (layer F.Cu) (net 26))
 (segment (start 108.774 79.719) (end 108.774 80.219) (width 0.3048) (layer F.Cu) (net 26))
 (segment (start 109.108322 83.219) (end 106.524 83.219) (width 0.3048) (layer F.Cu) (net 26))
 (segment (start 109.358322 83.469) (end 109.108322 83.219) (width 0.3048) (layer F.Cu) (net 26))
 (segment (start 114.024 83.469) (end 109.358322 83.469) (width 0.3048) (layer F.Cu) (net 26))
 (via (at 157.024 82.969) (size 0.6) (drill 0.4) (layers F.Cu B.Cu) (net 27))
 (segment (start 156.274 82.219) (end 157.024 82.969) (width 0.254) (layer F.Cu) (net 27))
 (segment (start 156.024 82.219) (end 156.274 82.219) (width 0.254) (layer F.Cu) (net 27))
 (segment (start 151.524 84.969) (end 149.896999 83.341999) (width 0.254) (layer B.Cu) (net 27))
 (segment (start 155.024 84.969) (end 151.524 84.969) (width 0.254) (layer B.Cu) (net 27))
 (segment (start 157.024 82.969) (end 155.024 84.969) (width 0.254) (layer B.Cu) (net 27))
 (segment (start 149.896999 83.341999) (end 147.651001 83.341999) (width 0.254) (layer B.Cu) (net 27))
 (segment (start 147.651001 83.341999) (end 146.274 84.719) (width 0.254) (layer B.Cu) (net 27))
 (segment (start 138.374 84.719) (end 136.949 83.294) (width 0.254) (layer B.Cu) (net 27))
 (segment (start 146.274 84.719) (end 138.374 84.719) (width 0.254) (layer B.Cu) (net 27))
 (segment (start 136.949 83.294) (end 136.274 82.619) (width 0.254) (layer B.Cu) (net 27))
 (segment (start 137.874 84.219) (end 136.949 83.294) (width 0.254) (layer B.Cu) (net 27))
 (segment (start 156.024 84.219) (end 156.024 84.469) (width 0.2) (layer F.Cu) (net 28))
 (segment (start 144.924 82.619) (end 145.774 83.469) (width 0.3048) (layer B.Cu) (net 28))
 (via (at 145.774 83.469) (size 0.6) (drill 0.4) (layers F.Cu B.Cu) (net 28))
 (segment (start 144.274 82.619) (end 144.924 82.619) (width 0.3048) (layer B.Cu) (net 28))
 (segment (start 147.95101 85.64601) (end 145.774 83.469) (width 0.254) (layer F.Cu) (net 28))
 (segment (start 155.59699 85.64601) (end 147.95101 85.64601) (width 0.254) (layer F.Cu) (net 28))
 (segment (start 156.024 85.219) (end 155.59699 85.64601) (width 0.254) (layer F.Cu) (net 28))
 (segment (start 156.024 84.219) (end 156.024 85.219) (width 0.254) (layer F.Cu) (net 28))
 (via (at 153.024 84.219) (size 0.6) (drill 0.4) (layers F.Cu B.Cu) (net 29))
 (segment (start 152.024 84.219) (end 153.024 84.219) (width 0.254) (layer F.Cu) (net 29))
 (segment (start 153.024 83.369) (end 152.274 82.619) (width 0.254) (layer B.Cu) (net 29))
 (segment (start 153.024 84.219) (end 153.024 83.369) (width 0.254) (layer B.Cu) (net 29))
 (segment (start 117.289 81.219) (end 117.289 79.234) (width 0.4064) (layer F.Cu) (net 1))
 (segment (start 117.289 81.219) (end 117.289 79.734) (width 0.4064) (layer F.Cu) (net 1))
 (segment (start 117.289 79.734) (end 114.774 77.219) (width 0.4064) (layer F.Cu) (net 1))
 (segment (start 104.774 77.219) (end 103.274 78.719) (width 0.4064) (layer F.Cu) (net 1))
 (segment (start 114.774 77.219) (end 104.774 77.219) (width 0.4064) (layer F.Cu) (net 1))
 (segment (start 148.724 80.419) (end 149.574 80.419) (width 0.2) (layer F.Cu) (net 6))
 (via (at 149.774 79.2158) (size 0.6) (drill 0.4) (layers F.Cu B.Cu) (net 6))
 (segment (start 149.774 80.219) (end 149.774 79.2158) (width 0.2) (layer F.Cu) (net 6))
 (segment (start 149.574 80.419) (end 149.774 80.219) (width 0.2) (layer F.Cu) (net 6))
 (segment (start 149.774 79.2158) (end 149.774 78.719) (width 0.3048) (layer B.Cu) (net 6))
 (segment (start 149.774 78.719) (end 149.024 77.969) (width 0.3048) (layer B.Cu) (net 6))
 (segment (start 113.274 78.219) (end 113.524 77.969) (width 0.3048) (layer F.Cu) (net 6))
 (via (at 113.524 77.969) (size 0.6) (drill 0.4) (layers F.Cu B.Cu) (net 6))
 (segment (start 108.774 78.219) (end 113.274 78.219) (width 0.3048) (layer F.Cu) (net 6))
 (segment (start 149.024 77.969) (end 113.524 77.969) (width 0.3048) (layer B.Cu) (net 6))
 (via (at 148.774 78.969) (size 0.6) (drill 0.4) (layers F.Cu B.Cu) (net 7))
 (segment (start 148.074 79.019) (end 148.124 78.969) (width 0.2) (layer F.Cu) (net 7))
 (segment (start 148.124 78.969) (end 148.774 78.969) (width 0.2) (layer F.Cu) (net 7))
 (segment (start 148.074 79.769) (end 148.074 79.019) (width 0.2) (layer F.Cu) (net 7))
 (segment (start 108.774 84.219) (end 108.774 84.719) (width 0.3048) (layer F.Cu) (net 7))
 (via (at 102.274 85.469) (size 0.6) (drill 0.4) (layers F.Cu B.Cu) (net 7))
 (segment (start 108.024 85.469) (end 102.274 85.469) (width 0.3048) (layer F.Cu) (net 7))
 (segment (start 108.774 84.719) (end 108.024 85.469) (width 0.3048) (layer F.Cu) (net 7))
 (segment (start 102.524 80.969) (end 102.524 79.25475) (width 0.3048) (layer B.Cu) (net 7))
 (segment (start 101.774 81.719) (end 102.524 80.969) (width 0.3048) (layer B.Cu) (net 7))
 (segment (start 101.774 84.969) (end 101.774 81.719) (width 0.3048) (layer B.Cu) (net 7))
 (segment (start 102.274 85.469) (end 101.774 84.969) (width 0.3048) (layer B.Cu) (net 7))
 (segment (start 103.05975 78.719) (end 103.041875 78.736875) (width 0.3048) (layer B.Cu) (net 7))
 (segment (start 148.524 78.719) (end 103.05975 78.719) (width 0.3048) (layer B.Cu) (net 7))
 (segment (start 148.774 78.969) (end 148.524 78.719) (width 0.3048) (layer B.Cu) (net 7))
 (segment (start 102.524 79.25475) (end 103.041875 78.736875) (width 0.3048) (layer B.Cu) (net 7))
 (via (at 105.774 82.719) (size 0.6) (drill 0.4) (layers F.Cu B.Cu) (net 14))
 (segment (start 106.274 82.219) (end 105.774 82.719) (width 0.3048) (layer F.Cu) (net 14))
 (segment (start 107.274 82.219) (end 106.274 82.219) (width 0.3048) (layer F.Cu) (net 14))
 (segment (start 106.37881 82.11419) (end 105.774 82.719) (width 0.3048) (layer B.Cu) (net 14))
 (segment (start 110.37881 82.11419) (end 106.37881 82.11419) (width 0.3048) (layer B.Cu) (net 14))
 (segment (start 145.824 81.219) (end 145.774 81.219) (width 0.2) (layer F.Cu) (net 14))
 (segment (start 110.82601 81.66699) (end 110.37881 82.11419) (width 0.254) (layer B.Cu) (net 14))
 (segment (start 142.703343 81.66699) (end 110.82601 81.66699) (width 0.254) (layer B.Cu) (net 14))
 (segment (start 142.774 81.969) (end 142.703343 81.66699) (width 0.254) (layer B.Cu) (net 14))
 (segment (start 143.679843 81.219) (end 145.824 81.219) (width 0.2) (layer F.Cu) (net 14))
 (segment (start 142.774 81.969) (end 143.679843 81.219) (width 0.2) (layer F.Cu) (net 14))
 (via (at 142.774 81.969) (size 0.6) (drill 0.4) (layers F.Cu B.Cu) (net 14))
 (via (at 109.774 81.219) (size 0.6) (drill 0.4) (layers F.Cu B.Cu) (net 13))
 (segment (start 109.86798 81.31298) (end 109.774 81.219) (width 0.254) (layer B.Cu) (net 13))
 (segment (start 109.774 81.219) (end 107.774 81.219) (width 0.254) (layer F.Cu) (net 13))
 (segment (start 107.274 80.719) (end 107.274 80.219) (width 0.254) (layer F.Cu) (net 13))
 (segment (start 107.774 81.219) (end 107.274 80.719) (width 0.254) (layer F.Cu) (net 13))
 (segment (start 143.124 80.819) (end 145.824 80.819) (width 0.2) (layer F.Cu) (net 13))
 (segment (start 142.774 80.719) (end 143.124 80.819) (width 0.2) (layer F.Cu) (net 13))
 (segment (start 110.024 81.219) (end 109.774 81.219) (width 0.254) (layer B.Cu) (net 13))
 (segment (start 142.774 80.969) (end 110.274 80.969) (width 0.254) (layer B.Cu) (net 13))
 (segment (start 142.774 80.719) (end 142.774 80.969) (width 0.254) (layer B.Cu) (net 13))
 (segment (start 110.274 80.969) (end 110.024 81.219) (width 0.254) (layer B.Cu) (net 13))
 (via (at 142.774 80.719) (size 0.6) (drill 0.4) (layers F.Cu B.Cu) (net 13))
 (via (at 153.774 81.219) (size 0.6) (drill 0.4) (layers F.Cu B.Cu) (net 15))
 (segment (start 153.774 81.219) (end 154.274 81.219) (width 0.254) (layer F.Cu) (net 15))
 (segment (start 154.524 81.469) (end 154.524 82.219) (width 0.254) (layer F.Cu) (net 15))
 (segment (start 154.274 81.219) (end 154.524 81.469) (width 0.254) (layer F.Cu) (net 15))
 (segment (start 145.824 81.619) (end 144.874 81.619) (width 0.2) (layer F.Cu) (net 15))
 (via (at 143.024 83.469) (size 0.6) (drill 0.4) (layers F.Cu B.Cu) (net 15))
 (segment (start 144.874 81.619) (end 143.024 83.469) (width 0.2) (layer F.Cu) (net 15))
 (segment (start 143.024 83.469) (end 143.774 84.219) (width 0.254) (layer B.Cu) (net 15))
 (segment (start 145.951962 84.219) (end 148.951962 81.219) (width 0.254) (layer B.Cu) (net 15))
 (segment (start 143.774 84.219) (end 145.951962 84.219) (width 0.254) (layer B.Cu) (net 15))
 (segment (start 148.951962 81.219) (end 153.774 81.219) (width 0.254) (layer B.Cu) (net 15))
 (segment (start 148.724 81.619) (end 150.174 81.619) (width 0.2) (layer F.Cu) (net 4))
 (segment (start 150.174 81.619) (end 151.524 82.969) (width 0.2) (layer F.Cu) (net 4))
 (segment (start 153.274 82.969) (end 154.524 84.219) (width 0.2) (layer F.Cu) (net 4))
 (segment (start 151.524 82.969) (end 153.274 82.969) (width 0.2) (layer F.Cu) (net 4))
 (segment (start 148.724 82.019) (end 149.824 82.019) (width 0.2) (layer F.Cu) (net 3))
 (segment (start 150.524 82.719) (end 150.524 84.219) (width 0.2) (layer F.Cu) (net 3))
 (segment (start 149.824 82.019) (end 150.524 82.719) (width 0.2) (layer F.Cu) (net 3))
 (segment (start 159.699 79.419) (end 159.699 83.019) (width 0.3048) (layer F.Cu) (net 21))
 (via (at 148.774 83.969) (size 0.6) (drill 0.4) (layers F.Cu B.Cu) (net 21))
 (segment (start 148.074 83.269) (end 148.774 83.969) (width 0.2) (layer F.Cu) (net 21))
 (segment (start 148.074 82.669) (end 148.074 83.269) (width 0.2) (layer F.Cu) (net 21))
 (segment (start 148.774 83.969) (end 150.024 85.219) (width 0.254) (layer B.Cu) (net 21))
 (via (at 157.024 85.469) (size 0.6) (drill 0.4) (layers F.Cu B.Cu) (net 21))
 (segment (start 150.274 85.469) (end 157.024 85.469) (width 0.254) (layer B.Cu) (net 21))
 (segment (start 150.024 85.219) (end 150.274 85.469) (width 0.254) (layer B.Cu) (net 21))
 (segment (start 157.024 85.469) (end 158.274 85.469) (width 0.254) (layer F.Cu) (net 21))
 (segment (start 159.699 84.044) (end 159.699 83.019) (width 0.254) (layer F.Cu) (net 21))
 (segment (start 158.274 85.469) (end 159.699 84.044) (width 0.254) (layer F.Cu) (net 21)))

